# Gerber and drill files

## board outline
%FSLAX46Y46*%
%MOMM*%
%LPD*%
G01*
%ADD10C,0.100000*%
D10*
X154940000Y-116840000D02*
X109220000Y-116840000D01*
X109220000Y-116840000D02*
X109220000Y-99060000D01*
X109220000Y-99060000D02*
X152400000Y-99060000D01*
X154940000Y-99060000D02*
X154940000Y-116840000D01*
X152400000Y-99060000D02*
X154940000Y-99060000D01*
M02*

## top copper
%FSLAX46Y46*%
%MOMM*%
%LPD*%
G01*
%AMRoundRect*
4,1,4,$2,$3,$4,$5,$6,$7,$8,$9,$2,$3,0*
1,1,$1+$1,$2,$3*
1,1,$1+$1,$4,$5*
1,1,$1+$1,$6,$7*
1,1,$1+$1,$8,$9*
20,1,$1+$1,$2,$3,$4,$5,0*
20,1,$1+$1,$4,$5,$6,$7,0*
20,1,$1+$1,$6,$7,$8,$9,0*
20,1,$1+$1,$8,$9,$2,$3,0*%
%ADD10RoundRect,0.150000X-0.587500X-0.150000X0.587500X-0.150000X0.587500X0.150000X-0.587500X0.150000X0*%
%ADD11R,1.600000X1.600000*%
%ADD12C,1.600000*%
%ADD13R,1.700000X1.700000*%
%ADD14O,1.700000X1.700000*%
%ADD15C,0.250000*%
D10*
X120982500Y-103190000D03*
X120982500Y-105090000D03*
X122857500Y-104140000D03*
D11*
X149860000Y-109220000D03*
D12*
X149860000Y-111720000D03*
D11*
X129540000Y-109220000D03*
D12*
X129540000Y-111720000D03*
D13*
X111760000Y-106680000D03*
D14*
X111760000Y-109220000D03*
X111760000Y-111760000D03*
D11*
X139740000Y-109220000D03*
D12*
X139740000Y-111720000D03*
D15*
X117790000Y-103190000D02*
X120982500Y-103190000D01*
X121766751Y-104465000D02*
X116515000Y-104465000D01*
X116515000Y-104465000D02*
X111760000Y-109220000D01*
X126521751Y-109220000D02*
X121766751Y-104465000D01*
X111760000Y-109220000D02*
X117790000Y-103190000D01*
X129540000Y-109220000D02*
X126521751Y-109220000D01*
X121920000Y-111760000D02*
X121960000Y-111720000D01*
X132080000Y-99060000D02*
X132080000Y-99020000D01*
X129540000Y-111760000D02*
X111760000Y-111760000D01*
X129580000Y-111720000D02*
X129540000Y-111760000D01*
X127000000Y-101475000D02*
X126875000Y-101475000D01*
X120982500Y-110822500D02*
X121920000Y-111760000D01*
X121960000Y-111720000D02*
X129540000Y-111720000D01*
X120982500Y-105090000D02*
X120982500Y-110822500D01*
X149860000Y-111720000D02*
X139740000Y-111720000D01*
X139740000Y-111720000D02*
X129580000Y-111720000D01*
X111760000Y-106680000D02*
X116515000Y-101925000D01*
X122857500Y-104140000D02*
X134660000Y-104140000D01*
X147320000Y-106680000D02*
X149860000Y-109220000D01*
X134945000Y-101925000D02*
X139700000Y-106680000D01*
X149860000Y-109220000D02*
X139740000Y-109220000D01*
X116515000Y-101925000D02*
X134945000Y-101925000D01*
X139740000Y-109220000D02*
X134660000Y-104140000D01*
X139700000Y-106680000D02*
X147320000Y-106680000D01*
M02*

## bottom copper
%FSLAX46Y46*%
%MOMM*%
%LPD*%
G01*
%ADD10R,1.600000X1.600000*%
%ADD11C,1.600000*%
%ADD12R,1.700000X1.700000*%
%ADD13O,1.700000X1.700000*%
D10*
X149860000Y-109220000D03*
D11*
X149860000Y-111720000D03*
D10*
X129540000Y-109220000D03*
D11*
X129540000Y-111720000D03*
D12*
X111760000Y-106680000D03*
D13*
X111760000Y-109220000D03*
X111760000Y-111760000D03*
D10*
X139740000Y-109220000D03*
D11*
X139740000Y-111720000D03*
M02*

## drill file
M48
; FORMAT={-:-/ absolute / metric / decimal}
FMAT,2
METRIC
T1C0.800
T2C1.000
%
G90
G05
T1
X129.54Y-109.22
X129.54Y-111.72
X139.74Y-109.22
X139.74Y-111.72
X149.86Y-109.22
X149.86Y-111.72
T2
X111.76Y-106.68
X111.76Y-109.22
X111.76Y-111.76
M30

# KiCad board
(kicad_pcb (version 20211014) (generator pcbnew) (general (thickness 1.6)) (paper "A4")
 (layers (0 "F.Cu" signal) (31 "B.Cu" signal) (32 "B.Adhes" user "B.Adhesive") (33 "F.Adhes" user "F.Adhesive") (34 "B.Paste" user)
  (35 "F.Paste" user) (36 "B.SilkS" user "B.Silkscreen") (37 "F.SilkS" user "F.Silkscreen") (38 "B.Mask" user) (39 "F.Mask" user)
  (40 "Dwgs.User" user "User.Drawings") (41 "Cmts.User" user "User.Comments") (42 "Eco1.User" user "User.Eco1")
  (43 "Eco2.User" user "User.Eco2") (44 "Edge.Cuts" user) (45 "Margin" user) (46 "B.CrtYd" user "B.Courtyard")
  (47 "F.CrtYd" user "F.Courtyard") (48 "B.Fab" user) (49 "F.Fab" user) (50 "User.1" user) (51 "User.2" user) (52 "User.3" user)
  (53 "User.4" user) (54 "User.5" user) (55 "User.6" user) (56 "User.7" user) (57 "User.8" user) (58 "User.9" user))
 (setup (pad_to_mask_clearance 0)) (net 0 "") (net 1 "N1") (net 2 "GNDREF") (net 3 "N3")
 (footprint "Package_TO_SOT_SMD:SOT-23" (layer "F.Cu") (at 121.92 104.14)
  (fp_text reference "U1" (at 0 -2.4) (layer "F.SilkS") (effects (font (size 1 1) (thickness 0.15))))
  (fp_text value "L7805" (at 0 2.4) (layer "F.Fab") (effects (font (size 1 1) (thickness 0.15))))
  (pad "1" smd roundrect (at -0.9375 -0.95) (size 1.475 0.6) (layers "F.Cu" "F.Paste" "F.Mask") (roundrect_rratio 0.25) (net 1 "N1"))
  (pad "2" smd roundrect (at -0.9375 0.95) (size 1.475 0.6) (layers "F.Cu" "F.Paste" "F.Mask") (roundrect_rratio 0.25) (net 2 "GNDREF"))
  (pad "3" smd roundrect (at 0.9375 0) (size 1.475 0.6) (layers "F.Cu" "F.Paste" "F.Mask") (roundrect_rratio 0.25) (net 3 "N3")))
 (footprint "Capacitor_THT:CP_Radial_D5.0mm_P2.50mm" (layer "F.Cu") (at 149.86 109.22 -90)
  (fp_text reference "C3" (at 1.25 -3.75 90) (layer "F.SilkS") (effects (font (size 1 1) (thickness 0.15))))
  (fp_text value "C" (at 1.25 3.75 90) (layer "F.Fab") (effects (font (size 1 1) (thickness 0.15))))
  (pad "1" thru_hole rect (at 0 0 270) (size 1.6 1.6) (drill 0.8) (layers *.Cu *.Mask) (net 3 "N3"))
  (pad "2" thru_hole circle (at 2.5 0 270) (size 1.6 1.6) (drill 0.8) (layers *.Cu *.Mask) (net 2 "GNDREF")))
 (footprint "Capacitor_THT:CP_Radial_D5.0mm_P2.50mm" (layer "F.Cu") (at 129.54 109.22 -90)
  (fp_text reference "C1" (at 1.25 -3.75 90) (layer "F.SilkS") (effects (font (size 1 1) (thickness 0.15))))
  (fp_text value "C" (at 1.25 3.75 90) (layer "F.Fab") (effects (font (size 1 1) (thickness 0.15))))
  (pad "1" thru_hole rect (at 0 0 270) (size 1.6 1.6) (drill 0.8) (layers *.Cu *.Mask) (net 1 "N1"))
  (pad "2" thru_hole circle (at 2.5 0 270) (size 1.6 1.6) (drill 0.8) (layers *.Cu *.Mask) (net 2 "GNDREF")))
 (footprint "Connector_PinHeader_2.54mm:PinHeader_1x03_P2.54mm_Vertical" (layer "F.Cu") (at 111.76 106.68)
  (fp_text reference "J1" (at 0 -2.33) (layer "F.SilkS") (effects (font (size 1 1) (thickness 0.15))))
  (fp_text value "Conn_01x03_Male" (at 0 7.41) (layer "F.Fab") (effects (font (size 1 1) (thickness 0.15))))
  (pad "1" thru_hole rect (at 0 0) (size 1.7 1.7) (drill 1) (layers *.Cu *.Mask) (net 3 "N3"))
  (pad "2" thru_hole oval (at 0 2.54) (size 1.7 1.7) (drill 1) (layers *.Cu *.Mask) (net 1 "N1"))
  (pad "3" thru_hole oval (at 0 5.08) (size 1.7 1.7) (drill 1) (layers *.Cu *.Mask) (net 2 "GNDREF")))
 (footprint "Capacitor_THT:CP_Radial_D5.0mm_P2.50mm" (layer "F.Cu") (at 139.74 109.22 -90)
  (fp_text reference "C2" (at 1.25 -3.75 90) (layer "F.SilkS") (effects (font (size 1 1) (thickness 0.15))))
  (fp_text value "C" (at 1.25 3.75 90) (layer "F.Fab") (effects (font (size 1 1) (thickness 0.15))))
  (pad "1" thru_hole rect (at 0 0 270) (size 1.6 1.6) (drill 0.8) (layers *.Cu *.Mask) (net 3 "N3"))
  (pad "2" thru_hole circle (at 2.5 0 270) (size 1.6 1.6) (drill 0.8) (layers *.Cu *.Mask) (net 2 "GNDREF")))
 (gr_line (start 154.94 116.84) (end 109.22 116.84) (layer "Edge.Cuts") (width 0.1))
 (gr_line (start 109.22 116.84) (end 109.22 99.06) (layer "Edge.Cuts") (width 0.1))
 (gr_line (start 109.22 99.06) (end 152.4 99.06) (layer "Edge.Cuts") (width 0.1))
 (gr_line (start 154.94 99.06) (end 154.94 116.84) (layer "Edge.Cuts") (width 0.1))
 (gr_line (start 152.4 99.06) (end 154.94 99.06) (layer "Edge.Cuts") (width 0.1))
 (segment (start 117.79 103.19) (end 120.9825 103.19) (width 0.25) (layer "F.Cu") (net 1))
 (segment (start 121.766751 104.465) (end 116.515 104.465) (width 0.25) (layer "F.Cu") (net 1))
 (segment (start 116.515 104.465) (end 111.76 109.22) (width 0.25) (layer "F.Cu") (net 1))
 (segment (start 126.521751 109.22) (end 121.766751 104.465) (width 0.25) (layer "F.Cu") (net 1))
 (segment (start 111.76 109.22) (end 117.79 103.19) (width 0.25) (layer "F.Cu") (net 1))
 (segment (start 129.54 109.22) (end 126.521751 109.22) (width 0.25) (layer "F.Cu") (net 1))
 (segment (start 121.92 111.76) (end 121.96 111.72) (width 0.25) (layer "F.Cu") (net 2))
 (segment (start 132.08 99.06) (end 132.08 99.02) (width 0.25) (layer "F.Cu") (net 2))
 (segment (start 129.54 111.76) (end 111.76 111.76) (width 0.25) (layer "F.Cu") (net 2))
 (segment (start 129.58 111.72) (end 129.54 111.76) (width 0.25) (layer "F.Cu") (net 2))
 (segment (start 127 101.475) (end 126.875 101.475) (width 0.25) (layer "F.Cu") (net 2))
 (segment (start 120.9825 110.8225) (end 121.92 111.76) (width 0.25) (layer "F.Cu") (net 2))
 (segment (start 121.96 111.72) (end 129.54 111.72) (width 0.25) (layer "F.Cu") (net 2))
 (segment (start 120.9825 105.09) (end 120.9825 110.8225) (width 0.25) (layer "F.Cu") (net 2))
 (segment (start 149.86 111.72) (end 139.74 111.72) (width 0.25) (layer "F.Cu") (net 2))
 (segment (start 139.74 111.72) (end 129.58 111.72) (width 0.25) (layer "F.Cu") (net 2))
 (segment (start 111.76 106.68) (end 116.515 101.925) (width 0.25) (layer "F.Cu") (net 3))
 (segment (start 122.8575 104.14) (end 134.66 104.14) (width 0.25) (layer "F.Cu") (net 3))
 (segment (start 147.32 106.68) (end 149.86 109.22) (width 0.25) (layer "F.Cu") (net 3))
 (segment (start 134.945 101.925) (end 139.7 106.68) (width 0.25) (layer "F.Cu") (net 3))
 (segment (start 149.86 109.22) (end 139.74 109.22) (width 0.25) (layer "F.Cu") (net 3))
 (segment (start 116.515 101.925) (end 134.945 101.925) (width 0.25) (layer "F.Cu") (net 3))
 (segment (start 139.74 109.22) (end 134.66 104.14) (width 0.25) (layer "F.Cu") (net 3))
 (segment (start 139.7 106.68) (end 147.32 106.68) (width 0.25) (layer "F.Cu") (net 3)))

